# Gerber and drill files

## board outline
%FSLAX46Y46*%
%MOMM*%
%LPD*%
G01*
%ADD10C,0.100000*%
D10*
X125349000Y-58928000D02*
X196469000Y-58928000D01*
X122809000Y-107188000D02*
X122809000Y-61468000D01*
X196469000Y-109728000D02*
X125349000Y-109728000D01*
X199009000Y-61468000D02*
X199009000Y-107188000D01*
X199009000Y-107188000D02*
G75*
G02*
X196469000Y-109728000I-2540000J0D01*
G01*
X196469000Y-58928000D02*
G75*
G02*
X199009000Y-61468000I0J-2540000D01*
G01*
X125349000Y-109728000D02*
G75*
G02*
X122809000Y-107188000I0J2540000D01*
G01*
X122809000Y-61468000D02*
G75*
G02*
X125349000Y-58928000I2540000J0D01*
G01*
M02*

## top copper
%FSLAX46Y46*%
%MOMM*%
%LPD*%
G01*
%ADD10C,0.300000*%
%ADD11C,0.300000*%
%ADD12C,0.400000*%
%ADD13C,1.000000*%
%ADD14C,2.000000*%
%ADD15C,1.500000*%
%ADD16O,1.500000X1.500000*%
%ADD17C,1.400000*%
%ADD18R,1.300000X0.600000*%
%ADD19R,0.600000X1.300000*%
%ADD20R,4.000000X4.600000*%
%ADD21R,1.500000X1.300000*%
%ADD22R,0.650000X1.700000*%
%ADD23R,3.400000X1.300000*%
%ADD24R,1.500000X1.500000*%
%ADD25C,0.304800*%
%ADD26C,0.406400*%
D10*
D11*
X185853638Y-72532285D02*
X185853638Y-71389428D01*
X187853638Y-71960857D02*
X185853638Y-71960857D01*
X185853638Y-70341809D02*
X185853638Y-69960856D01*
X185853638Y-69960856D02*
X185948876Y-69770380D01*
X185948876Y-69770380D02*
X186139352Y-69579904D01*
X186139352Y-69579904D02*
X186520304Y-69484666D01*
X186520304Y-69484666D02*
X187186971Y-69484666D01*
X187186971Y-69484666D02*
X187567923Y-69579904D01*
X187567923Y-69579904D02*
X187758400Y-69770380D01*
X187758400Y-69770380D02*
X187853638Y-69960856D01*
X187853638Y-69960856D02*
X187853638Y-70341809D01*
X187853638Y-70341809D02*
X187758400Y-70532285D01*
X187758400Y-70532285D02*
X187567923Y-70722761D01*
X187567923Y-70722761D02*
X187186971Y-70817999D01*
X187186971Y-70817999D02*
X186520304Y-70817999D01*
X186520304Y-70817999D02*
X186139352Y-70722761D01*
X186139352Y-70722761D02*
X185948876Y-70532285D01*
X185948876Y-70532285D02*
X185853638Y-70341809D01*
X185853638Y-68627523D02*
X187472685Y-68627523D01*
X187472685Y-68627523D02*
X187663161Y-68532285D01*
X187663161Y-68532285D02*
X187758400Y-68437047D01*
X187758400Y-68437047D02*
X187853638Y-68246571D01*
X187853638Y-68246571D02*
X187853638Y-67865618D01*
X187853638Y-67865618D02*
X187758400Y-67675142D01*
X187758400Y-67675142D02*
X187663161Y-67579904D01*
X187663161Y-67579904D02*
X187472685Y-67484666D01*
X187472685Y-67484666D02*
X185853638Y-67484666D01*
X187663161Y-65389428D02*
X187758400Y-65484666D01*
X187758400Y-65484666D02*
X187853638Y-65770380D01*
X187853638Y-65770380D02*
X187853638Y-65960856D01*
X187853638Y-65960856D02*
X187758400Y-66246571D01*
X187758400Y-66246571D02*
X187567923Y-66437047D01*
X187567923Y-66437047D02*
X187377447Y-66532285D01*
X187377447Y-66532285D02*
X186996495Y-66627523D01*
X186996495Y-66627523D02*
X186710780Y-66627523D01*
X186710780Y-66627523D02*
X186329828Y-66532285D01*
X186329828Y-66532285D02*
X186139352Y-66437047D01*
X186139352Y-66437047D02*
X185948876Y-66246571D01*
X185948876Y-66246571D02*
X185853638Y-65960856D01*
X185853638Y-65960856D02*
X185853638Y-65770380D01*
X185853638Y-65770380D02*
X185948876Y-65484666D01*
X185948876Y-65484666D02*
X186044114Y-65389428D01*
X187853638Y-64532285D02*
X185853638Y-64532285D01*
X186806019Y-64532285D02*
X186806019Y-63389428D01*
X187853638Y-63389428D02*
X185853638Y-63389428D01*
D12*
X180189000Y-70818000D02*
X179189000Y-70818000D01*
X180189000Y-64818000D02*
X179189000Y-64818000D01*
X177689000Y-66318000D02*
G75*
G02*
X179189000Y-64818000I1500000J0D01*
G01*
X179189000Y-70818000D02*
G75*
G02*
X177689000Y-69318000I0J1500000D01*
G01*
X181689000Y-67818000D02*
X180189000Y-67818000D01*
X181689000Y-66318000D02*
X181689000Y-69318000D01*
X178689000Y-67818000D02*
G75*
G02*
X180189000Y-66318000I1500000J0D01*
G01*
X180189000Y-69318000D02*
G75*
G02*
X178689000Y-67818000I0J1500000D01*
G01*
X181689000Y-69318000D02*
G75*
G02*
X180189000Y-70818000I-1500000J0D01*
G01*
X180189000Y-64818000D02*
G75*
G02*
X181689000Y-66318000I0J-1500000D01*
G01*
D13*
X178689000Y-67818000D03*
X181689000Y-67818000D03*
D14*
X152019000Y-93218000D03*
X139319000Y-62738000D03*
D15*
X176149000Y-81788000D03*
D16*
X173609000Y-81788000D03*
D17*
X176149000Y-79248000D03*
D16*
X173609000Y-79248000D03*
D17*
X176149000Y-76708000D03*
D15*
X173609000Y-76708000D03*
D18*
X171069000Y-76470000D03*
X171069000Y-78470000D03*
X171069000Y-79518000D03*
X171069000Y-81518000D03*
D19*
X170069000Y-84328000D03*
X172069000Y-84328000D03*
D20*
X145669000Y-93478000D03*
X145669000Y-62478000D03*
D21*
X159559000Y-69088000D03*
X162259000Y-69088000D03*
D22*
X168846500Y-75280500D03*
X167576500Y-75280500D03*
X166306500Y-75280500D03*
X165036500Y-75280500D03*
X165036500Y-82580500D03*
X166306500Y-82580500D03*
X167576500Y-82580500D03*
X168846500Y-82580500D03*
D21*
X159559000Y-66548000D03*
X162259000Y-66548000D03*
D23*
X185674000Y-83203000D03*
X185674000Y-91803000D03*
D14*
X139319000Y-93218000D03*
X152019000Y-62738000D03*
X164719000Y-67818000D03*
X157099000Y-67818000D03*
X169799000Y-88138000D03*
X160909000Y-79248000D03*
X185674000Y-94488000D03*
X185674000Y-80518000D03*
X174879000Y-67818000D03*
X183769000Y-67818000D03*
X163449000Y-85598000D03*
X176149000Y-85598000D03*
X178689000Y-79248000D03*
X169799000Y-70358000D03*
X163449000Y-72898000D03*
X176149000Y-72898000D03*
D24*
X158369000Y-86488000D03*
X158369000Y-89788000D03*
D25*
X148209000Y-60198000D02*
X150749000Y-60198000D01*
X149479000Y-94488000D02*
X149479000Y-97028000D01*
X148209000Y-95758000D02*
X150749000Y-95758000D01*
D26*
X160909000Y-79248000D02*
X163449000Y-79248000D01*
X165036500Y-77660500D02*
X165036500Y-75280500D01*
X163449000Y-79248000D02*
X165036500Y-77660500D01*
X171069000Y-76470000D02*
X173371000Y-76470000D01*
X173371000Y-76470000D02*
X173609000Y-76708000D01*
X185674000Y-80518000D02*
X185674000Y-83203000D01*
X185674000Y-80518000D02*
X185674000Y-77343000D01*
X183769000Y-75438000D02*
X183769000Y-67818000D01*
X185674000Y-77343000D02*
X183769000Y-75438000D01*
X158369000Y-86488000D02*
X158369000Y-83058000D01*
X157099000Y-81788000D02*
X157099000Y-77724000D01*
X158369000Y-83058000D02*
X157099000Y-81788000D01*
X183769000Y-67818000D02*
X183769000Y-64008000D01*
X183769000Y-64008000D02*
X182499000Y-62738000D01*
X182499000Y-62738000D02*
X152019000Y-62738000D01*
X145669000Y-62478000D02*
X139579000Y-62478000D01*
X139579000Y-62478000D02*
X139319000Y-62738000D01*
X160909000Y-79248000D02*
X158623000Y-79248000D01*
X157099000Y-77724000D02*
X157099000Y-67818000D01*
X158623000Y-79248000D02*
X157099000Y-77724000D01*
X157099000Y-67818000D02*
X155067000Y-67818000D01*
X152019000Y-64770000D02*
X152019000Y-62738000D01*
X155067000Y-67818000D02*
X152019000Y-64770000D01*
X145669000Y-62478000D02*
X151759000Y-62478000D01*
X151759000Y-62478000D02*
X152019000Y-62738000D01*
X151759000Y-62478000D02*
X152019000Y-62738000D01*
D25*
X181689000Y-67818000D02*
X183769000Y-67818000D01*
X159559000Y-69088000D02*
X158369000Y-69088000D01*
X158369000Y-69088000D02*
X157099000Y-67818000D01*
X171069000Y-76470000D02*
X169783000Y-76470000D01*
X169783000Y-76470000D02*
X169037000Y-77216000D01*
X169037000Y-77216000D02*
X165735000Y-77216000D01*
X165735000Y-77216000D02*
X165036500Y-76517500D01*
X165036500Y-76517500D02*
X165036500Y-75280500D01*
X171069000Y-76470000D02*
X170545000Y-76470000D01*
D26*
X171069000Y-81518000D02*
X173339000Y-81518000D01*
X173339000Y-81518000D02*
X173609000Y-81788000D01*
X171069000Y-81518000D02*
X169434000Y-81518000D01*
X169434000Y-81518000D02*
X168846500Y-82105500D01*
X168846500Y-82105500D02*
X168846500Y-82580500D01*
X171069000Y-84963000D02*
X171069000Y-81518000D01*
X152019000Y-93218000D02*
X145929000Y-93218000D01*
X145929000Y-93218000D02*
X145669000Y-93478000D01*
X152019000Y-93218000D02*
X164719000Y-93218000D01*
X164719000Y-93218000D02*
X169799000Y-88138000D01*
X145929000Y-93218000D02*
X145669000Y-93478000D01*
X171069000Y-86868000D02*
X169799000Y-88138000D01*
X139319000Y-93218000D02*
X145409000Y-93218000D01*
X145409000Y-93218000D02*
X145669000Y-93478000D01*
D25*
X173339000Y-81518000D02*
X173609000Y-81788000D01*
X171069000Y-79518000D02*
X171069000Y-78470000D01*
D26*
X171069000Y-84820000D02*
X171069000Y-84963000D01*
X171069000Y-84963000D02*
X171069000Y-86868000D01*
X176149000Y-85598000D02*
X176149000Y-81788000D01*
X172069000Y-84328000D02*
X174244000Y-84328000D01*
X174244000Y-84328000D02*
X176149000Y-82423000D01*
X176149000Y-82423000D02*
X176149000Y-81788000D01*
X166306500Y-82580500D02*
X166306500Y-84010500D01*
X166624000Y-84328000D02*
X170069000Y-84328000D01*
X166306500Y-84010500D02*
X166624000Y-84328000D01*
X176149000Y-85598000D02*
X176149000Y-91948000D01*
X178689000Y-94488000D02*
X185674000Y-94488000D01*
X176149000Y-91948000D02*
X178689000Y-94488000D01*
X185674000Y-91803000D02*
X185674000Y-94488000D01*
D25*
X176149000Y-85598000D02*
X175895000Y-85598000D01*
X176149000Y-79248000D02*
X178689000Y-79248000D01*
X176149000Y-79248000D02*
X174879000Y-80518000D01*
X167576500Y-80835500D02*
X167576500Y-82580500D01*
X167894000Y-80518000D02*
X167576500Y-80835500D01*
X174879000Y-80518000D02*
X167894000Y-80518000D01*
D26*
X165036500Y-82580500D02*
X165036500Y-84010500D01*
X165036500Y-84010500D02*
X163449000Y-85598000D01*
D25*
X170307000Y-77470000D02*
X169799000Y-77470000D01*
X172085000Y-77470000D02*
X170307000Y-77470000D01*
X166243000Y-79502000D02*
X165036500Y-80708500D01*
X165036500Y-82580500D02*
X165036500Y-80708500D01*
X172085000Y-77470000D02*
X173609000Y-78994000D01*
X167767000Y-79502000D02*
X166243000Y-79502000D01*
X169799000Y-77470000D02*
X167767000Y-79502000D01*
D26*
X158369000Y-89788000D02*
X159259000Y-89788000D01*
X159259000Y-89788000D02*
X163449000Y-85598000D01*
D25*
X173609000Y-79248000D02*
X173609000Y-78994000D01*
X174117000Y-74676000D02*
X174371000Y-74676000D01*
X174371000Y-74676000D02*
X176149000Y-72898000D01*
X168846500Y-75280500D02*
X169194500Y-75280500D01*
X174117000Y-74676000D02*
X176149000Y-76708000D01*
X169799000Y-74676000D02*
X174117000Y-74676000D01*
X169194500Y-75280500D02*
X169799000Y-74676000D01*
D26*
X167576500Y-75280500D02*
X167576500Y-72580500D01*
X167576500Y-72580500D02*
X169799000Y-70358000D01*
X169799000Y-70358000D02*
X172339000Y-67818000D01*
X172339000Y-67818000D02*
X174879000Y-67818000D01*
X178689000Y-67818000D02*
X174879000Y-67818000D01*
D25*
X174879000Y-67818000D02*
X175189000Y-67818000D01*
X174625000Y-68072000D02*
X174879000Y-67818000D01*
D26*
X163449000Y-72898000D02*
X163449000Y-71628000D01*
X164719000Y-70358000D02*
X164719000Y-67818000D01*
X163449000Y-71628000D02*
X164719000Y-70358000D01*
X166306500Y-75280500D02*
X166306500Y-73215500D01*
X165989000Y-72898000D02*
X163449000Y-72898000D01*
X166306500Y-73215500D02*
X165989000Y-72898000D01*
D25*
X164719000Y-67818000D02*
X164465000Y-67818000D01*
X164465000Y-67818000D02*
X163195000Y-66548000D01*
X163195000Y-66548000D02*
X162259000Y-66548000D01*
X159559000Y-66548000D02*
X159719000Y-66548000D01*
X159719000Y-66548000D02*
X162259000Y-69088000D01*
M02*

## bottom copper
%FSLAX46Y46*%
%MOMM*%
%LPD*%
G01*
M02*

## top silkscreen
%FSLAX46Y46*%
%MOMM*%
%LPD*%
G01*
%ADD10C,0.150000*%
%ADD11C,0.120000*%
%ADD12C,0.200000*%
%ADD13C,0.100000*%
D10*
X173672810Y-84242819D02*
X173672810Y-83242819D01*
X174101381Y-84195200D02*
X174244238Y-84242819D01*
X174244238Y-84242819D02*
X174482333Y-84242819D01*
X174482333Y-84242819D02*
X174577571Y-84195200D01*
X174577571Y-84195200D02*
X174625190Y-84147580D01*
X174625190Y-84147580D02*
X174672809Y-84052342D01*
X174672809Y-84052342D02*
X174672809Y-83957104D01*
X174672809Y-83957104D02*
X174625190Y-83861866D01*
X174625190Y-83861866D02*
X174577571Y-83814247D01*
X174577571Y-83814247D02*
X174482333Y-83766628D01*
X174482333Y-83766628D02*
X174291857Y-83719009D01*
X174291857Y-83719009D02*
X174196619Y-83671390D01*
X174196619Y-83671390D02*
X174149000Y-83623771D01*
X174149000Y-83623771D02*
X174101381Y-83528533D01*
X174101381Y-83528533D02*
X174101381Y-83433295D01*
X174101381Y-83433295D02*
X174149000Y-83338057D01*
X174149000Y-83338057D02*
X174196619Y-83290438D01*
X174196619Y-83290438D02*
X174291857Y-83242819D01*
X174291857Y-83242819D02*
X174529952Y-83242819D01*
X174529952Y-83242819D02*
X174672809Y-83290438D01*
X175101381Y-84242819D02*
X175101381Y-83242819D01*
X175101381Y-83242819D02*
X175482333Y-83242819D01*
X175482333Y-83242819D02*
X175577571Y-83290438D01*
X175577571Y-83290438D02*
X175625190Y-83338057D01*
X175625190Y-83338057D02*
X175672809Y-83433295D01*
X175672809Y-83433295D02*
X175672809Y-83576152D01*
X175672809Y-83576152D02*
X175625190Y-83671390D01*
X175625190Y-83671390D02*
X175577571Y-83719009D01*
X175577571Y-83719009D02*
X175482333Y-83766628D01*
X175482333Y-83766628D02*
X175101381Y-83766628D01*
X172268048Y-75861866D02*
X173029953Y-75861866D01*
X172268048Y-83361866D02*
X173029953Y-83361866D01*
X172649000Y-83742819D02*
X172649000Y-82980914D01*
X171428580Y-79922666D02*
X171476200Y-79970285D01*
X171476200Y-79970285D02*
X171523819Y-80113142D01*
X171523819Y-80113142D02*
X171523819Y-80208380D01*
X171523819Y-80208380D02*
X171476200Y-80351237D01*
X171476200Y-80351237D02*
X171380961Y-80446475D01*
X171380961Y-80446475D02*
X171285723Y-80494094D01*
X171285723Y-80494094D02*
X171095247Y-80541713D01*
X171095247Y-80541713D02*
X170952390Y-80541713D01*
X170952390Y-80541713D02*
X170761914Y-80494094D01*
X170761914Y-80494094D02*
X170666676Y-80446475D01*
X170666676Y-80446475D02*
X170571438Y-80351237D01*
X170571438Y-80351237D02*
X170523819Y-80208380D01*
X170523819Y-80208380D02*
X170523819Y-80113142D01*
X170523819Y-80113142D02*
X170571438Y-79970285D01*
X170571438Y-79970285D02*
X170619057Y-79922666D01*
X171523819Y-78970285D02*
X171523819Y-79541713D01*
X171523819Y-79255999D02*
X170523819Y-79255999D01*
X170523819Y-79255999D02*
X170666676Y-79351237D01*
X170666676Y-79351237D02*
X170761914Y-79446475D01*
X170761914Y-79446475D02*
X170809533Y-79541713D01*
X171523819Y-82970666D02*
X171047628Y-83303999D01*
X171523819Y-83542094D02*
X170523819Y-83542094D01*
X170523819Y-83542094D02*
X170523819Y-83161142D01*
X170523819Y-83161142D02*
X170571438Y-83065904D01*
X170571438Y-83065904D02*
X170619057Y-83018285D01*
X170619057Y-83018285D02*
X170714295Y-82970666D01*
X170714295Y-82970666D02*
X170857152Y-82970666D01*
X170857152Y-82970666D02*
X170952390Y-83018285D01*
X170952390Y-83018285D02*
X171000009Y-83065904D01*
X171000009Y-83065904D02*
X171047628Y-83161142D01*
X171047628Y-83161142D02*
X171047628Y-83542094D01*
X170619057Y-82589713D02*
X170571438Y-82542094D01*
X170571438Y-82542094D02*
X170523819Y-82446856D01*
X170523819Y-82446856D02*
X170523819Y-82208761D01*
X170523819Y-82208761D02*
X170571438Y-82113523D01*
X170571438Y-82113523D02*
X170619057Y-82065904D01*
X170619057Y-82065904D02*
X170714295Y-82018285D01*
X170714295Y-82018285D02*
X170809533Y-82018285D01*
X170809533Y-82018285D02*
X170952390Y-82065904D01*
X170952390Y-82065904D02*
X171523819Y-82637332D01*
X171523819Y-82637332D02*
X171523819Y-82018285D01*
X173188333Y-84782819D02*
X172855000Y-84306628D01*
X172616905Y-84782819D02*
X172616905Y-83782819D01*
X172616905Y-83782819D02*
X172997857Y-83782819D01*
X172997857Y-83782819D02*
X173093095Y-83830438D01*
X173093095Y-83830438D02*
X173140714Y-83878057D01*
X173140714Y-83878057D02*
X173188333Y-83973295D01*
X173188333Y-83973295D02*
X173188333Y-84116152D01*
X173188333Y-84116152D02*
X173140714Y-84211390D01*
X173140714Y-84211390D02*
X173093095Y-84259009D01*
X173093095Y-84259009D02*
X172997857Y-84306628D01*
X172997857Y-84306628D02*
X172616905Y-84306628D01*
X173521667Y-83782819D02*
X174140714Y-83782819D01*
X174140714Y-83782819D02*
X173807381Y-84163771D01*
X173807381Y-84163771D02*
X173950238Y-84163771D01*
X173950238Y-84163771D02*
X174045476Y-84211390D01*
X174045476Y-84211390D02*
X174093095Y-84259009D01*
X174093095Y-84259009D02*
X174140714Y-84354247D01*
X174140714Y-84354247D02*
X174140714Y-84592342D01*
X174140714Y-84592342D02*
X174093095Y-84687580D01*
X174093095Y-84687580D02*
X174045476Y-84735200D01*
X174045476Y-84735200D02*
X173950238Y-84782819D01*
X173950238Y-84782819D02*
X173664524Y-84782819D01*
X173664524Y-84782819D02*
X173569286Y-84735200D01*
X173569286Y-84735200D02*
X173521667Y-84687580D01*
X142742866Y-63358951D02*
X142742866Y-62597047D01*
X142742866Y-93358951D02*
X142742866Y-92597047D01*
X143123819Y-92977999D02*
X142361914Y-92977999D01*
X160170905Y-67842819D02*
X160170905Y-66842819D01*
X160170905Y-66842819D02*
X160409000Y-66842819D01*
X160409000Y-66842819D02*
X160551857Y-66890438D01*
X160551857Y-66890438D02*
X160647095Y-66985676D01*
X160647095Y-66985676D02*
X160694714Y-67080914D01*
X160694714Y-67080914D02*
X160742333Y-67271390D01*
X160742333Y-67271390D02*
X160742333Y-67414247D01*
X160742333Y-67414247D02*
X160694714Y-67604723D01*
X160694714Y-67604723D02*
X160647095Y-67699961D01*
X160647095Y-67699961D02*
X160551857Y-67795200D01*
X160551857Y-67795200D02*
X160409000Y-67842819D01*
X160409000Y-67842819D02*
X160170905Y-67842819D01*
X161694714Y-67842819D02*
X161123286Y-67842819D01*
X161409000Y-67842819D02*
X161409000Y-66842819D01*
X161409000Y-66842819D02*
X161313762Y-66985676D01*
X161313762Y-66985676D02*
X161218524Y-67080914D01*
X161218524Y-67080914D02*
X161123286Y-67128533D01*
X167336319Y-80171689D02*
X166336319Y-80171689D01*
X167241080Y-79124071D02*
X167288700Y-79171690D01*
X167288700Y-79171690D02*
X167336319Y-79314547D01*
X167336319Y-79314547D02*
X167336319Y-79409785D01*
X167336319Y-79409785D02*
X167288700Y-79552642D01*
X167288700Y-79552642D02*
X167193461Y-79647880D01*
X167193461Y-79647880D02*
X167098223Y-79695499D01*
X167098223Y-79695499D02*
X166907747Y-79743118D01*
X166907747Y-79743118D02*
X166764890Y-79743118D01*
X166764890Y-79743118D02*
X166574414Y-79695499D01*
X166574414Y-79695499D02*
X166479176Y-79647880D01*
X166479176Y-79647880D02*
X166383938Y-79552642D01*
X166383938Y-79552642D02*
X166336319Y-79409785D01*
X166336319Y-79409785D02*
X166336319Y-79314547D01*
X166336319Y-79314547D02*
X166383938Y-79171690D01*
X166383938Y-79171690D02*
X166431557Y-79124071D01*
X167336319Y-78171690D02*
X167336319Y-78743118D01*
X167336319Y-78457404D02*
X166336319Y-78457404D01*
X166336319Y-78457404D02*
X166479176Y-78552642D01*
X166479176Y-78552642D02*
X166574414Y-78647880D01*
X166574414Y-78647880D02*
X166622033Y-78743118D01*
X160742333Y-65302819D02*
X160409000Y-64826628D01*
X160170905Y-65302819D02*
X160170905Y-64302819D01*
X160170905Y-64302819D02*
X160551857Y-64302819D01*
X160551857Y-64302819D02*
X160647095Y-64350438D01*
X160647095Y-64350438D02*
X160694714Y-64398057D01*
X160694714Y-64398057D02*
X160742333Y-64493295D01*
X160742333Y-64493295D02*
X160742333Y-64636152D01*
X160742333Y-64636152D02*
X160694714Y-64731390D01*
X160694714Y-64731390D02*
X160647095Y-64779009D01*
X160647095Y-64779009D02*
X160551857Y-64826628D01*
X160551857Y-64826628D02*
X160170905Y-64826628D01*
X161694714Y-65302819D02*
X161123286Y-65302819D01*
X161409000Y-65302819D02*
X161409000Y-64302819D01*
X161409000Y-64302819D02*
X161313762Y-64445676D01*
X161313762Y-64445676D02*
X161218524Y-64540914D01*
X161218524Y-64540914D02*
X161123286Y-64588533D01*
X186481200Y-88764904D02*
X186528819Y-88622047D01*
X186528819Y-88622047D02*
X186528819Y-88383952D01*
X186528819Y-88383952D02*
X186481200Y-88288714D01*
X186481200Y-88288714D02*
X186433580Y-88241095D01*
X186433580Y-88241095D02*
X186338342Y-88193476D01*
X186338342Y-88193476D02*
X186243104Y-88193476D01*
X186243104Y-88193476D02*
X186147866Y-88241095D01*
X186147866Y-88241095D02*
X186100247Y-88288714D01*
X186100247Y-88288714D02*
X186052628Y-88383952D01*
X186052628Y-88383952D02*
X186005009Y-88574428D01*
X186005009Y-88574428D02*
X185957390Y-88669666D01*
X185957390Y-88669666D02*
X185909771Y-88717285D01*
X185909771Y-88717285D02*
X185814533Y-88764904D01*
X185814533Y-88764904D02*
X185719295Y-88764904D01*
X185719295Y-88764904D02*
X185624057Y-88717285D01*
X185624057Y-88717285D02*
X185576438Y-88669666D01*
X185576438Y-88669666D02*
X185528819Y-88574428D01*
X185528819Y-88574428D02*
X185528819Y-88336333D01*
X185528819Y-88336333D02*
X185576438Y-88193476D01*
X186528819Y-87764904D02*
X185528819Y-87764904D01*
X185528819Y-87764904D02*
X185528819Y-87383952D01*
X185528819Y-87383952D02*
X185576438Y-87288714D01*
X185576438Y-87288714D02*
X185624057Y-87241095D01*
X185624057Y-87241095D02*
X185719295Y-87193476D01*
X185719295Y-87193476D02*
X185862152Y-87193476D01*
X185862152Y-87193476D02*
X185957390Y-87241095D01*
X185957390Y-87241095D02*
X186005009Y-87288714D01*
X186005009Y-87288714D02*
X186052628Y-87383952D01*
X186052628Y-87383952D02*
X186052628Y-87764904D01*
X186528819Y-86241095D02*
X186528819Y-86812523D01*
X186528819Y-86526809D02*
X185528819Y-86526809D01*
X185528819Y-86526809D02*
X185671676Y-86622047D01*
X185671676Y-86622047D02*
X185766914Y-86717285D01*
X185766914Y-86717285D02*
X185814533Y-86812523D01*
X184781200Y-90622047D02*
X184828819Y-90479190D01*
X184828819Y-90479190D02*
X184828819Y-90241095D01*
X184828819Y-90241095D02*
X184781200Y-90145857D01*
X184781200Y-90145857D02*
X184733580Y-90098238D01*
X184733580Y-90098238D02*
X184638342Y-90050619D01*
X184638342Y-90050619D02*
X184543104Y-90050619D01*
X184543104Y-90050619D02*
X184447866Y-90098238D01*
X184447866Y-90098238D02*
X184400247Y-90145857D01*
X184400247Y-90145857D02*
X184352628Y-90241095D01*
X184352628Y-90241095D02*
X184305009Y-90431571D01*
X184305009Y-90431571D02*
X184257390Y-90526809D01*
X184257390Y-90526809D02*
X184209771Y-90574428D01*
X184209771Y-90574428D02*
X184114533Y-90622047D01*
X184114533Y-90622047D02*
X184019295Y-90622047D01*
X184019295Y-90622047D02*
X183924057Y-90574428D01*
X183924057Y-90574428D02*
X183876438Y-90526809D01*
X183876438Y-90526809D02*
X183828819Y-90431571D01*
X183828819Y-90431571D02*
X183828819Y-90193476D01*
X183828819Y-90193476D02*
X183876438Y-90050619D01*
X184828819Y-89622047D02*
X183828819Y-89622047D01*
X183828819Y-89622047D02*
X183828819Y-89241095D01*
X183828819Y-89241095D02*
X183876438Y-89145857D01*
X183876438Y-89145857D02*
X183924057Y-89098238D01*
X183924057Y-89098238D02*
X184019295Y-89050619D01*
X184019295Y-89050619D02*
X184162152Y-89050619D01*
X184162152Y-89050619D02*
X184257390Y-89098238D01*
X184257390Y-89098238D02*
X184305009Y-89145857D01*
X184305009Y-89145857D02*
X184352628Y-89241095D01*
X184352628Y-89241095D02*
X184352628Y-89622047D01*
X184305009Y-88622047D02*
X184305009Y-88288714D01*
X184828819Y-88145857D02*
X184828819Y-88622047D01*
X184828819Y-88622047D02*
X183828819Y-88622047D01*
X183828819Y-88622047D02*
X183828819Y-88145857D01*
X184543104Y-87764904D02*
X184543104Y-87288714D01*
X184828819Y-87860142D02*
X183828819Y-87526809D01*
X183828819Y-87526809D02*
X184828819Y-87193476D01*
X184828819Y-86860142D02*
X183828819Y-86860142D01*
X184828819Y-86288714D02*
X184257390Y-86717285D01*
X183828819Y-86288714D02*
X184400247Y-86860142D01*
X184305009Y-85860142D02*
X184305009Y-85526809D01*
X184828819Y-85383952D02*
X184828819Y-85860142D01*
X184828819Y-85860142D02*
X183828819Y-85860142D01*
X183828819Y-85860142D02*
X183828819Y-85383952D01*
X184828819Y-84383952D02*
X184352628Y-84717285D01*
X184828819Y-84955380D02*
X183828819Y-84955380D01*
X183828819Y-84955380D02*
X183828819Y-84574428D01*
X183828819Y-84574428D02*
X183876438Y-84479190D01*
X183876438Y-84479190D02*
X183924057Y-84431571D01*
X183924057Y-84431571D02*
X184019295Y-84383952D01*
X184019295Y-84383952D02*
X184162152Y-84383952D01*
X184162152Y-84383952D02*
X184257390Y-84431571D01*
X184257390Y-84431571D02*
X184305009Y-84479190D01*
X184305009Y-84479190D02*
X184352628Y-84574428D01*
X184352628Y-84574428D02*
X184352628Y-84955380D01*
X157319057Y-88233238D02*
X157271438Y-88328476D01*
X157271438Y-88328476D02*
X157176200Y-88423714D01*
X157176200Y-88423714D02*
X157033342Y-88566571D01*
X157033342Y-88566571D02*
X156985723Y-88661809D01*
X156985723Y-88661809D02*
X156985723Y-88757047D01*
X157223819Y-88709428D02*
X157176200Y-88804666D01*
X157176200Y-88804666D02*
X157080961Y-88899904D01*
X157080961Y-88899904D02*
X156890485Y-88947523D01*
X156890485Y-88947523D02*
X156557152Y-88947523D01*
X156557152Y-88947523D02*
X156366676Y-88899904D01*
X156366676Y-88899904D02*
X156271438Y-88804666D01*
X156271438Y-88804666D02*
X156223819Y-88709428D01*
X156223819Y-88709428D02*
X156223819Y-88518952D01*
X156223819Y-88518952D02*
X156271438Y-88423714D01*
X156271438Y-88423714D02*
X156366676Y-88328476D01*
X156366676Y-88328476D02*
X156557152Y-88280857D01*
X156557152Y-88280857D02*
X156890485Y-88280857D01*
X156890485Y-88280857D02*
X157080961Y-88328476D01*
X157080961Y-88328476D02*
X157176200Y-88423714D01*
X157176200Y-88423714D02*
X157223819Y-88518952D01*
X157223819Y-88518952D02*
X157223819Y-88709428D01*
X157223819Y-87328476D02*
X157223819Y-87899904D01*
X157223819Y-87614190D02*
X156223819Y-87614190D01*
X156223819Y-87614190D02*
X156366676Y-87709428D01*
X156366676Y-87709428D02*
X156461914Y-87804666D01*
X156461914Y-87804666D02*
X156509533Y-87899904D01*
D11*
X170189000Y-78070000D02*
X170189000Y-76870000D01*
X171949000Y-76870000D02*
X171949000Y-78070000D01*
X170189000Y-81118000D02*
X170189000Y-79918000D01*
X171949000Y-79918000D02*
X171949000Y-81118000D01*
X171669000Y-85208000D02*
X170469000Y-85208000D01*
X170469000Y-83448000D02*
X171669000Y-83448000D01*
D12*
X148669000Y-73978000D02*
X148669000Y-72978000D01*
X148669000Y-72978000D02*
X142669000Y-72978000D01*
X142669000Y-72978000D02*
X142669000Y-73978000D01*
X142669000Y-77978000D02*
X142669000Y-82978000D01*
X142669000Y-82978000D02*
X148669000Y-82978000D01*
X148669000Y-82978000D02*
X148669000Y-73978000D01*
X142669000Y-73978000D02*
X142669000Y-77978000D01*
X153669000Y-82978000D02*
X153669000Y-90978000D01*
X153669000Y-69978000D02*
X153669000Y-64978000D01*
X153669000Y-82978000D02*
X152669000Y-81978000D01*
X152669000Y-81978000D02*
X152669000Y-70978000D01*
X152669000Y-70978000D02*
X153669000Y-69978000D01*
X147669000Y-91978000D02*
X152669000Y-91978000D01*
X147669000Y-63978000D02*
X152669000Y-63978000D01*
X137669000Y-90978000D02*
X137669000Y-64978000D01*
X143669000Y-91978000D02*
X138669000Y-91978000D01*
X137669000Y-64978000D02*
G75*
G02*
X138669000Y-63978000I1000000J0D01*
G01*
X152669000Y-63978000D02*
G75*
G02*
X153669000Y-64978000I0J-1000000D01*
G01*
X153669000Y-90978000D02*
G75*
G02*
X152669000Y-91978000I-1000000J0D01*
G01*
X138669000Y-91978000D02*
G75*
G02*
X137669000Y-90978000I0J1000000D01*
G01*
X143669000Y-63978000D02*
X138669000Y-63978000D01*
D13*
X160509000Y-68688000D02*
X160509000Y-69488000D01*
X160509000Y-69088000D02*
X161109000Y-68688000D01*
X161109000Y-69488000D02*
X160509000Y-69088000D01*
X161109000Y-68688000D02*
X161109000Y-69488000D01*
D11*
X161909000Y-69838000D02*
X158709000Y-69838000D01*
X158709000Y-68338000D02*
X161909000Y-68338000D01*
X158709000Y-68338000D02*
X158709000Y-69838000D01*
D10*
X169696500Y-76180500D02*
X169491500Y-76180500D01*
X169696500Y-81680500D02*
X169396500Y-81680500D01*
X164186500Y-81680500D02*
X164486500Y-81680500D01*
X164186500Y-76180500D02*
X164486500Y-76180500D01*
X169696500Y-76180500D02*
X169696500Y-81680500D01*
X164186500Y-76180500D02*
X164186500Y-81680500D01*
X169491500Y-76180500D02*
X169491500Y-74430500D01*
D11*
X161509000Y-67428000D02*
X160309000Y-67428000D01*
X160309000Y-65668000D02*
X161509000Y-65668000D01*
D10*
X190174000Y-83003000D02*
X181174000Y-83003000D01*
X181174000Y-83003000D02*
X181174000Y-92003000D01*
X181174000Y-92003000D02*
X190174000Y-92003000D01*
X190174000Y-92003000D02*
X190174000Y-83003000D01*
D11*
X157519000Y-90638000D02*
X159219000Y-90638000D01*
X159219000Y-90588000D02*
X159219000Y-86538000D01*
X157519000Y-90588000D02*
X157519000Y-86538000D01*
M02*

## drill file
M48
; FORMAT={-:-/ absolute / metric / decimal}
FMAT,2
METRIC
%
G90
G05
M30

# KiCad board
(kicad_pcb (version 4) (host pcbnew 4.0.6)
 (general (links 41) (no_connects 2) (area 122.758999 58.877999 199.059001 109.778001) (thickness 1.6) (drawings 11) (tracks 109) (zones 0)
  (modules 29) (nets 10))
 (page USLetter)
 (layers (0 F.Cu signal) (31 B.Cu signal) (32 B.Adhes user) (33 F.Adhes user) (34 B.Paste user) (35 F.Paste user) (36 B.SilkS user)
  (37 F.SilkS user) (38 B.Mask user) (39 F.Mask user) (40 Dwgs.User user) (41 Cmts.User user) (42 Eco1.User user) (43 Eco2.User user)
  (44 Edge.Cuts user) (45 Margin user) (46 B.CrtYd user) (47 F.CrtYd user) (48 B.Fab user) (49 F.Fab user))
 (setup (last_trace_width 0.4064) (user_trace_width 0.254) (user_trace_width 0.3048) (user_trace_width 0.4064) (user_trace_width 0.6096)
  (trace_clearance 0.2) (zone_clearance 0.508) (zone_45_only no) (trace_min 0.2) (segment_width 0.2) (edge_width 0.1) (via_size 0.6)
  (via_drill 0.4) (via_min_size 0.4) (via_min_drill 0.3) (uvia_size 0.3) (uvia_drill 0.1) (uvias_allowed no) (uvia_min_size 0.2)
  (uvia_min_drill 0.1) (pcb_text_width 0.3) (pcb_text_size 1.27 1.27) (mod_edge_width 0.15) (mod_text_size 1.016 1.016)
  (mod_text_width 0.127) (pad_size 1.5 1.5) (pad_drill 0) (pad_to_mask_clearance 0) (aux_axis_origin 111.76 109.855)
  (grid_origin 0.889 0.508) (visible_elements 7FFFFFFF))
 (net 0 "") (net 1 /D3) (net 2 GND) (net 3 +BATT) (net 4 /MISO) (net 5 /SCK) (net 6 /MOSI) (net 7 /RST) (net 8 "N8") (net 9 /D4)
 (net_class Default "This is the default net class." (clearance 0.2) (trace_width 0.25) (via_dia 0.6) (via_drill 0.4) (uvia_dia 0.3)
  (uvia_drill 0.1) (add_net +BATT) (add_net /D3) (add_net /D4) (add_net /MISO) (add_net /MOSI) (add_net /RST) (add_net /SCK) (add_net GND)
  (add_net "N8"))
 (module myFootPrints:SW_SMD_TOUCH (layer F.Cu) (at 178.689 67.818 270)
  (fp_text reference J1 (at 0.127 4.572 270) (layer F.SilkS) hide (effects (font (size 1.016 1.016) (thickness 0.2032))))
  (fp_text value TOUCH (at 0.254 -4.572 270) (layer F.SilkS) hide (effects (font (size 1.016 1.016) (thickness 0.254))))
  (fp_line (start 3 -1.5) (end 3 -0.5) (layer F.Cu) (width 0.4))
  (fp_line (start -3 -1.5) (end -3 -0.5) (layer F.Cu) (width 0.4))
  (fp_arc (start -1.5 -0.5) (end -1.5 1) (angle 90) (layer F.Cu) (width 0.4))
  (fp_arc (start 1.5 -0.5) (end 3 -0.5) (angle 90) (layer F.Cu) (width 0.4)) (fp_line (start 0 -3) (end 0 -1.5) (layer F.Cu) (width 0.4))
  (fp_line (start -1.5 -3) (end 1.5 -3) (layer F.Cu) (width 0.4))
  (fp_arc (start 0 -1.5) (end 0 0) (angle 90) (layer F.Cu) (width 0.4))
  (fp_arc (start 0 -1.5) (end 1.5 -1.5) (angle 90) (layer F.Cu) (width 0.4))
  (fp_arc (start 1.5 -1.5) (end 1.5 -3) (angle 90) (layer F.Cu) (width 0.4))
  (fp_arc (start -1.5 -1.5) (end -3 -1.5) (angle 90) (layer F.Cu) (width 0.4))
  (pad 2 smd circle (at 0 0 270) (size 1 1) (layers F.Cu) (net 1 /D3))
  (pad 1 smd circle (at 0 -3 270) (size 1 1) (layers F.Cu) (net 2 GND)))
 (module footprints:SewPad (layer F.Cu) (at 152.019 93.218)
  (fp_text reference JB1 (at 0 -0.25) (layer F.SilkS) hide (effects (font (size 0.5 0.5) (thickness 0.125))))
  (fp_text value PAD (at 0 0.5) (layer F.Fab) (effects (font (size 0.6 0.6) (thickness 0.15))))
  (pad 1 smd circle (at 0 0) (size 2 2) (layers F.Cu F.Mask) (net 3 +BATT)))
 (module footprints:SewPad (layer F.Cu) (at 139.319 62.738)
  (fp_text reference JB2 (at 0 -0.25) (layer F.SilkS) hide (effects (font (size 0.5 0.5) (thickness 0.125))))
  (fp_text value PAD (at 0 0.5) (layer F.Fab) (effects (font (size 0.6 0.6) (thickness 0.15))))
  (pad 1 smd circle (at 0 0) (size 2 2) (layers F.Cu F.Mask) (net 2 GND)))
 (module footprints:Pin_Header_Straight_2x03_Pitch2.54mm (layer F.Cu) (at 176.149 81.788 180)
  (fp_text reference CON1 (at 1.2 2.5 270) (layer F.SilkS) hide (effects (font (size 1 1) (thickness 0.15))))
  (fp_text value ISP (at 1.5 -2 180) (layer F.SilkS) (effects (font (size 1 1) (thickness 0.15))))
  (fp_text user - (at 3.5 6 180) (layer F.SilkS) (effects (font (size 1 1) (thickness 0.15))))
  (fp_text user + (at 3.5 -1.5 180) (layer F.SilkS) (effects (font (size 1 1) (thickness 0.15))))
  (pad 1 smd circle (at 0 0 180) (size 1.5 1.5) (layers F.Cu) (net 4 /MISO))
  (pad 2 smd oval (at 2.54 0 180) (size 1.5 1.5) (layers F.Cu) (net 3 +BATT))
  (pad 3 smd circle (at 0 2.54 180) (size 1.4 1.4) (layers F.Cu) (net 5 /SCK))
  (pad 4 smd oval (at 2.54 2.54 180) (size 1.5 1.5) (layers F.Cu) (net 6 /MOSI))
  (pad 5 smd circle (at 0 5.08 180) (size 1.4 1.4) (layers F.Cu) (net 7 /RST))
  (pad 6 smd circle (at 2.54 5.08 180) (size 1.5 1.5) (layers F.Cu) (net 2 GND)))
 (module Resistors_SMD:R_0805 (layer F.Cu) (at 171.069 77.47 270)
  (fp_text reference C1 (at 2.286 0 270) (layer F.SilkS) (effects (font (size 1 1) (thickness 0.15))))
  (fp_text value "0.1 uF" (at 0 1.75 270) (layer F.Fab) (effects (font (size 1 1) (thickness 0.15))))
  (fp_line (start 0.6 0.88) (end -0.6 0.88) (layer F.SilkS) (width 0.12))
  (fp_line (start -0.6 -0.88) (end 0.6 -0.88) (layer F.SilkS) (width 0.12))
  (pad 1 smd rect (at -1 0 270) (size 0.6 1.3) (layers F.Cu F.Paste F.Mask) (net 2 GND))
  (pad 2 smd rect (at 1 0 270) (size 0.6 1.3) (layers F.Cu F.Paste F.Mask) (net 3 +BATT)))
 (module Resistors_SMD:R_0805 (layer F.Cu) (at 171.069 80.518 270)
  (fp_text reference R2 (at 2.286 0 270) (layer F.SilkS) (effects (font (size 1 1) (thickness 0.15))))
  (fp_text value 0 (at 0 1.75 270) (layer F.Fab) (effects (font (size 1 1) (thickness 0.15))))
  (fp_line (start 0.6 0.88) (end -0.6 0.88) (layer F.SilkS) (width 0.12))
  (fp_line (start -0.6 -0.88) (end 0.6 -0.88) (layer F.SilkS) (width 0.12))
  (pad 1 smd rect (at -1 0 270) (size 0.6 1.3) (layers F.Cu F.Paste F.Mask) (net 3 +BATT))
  (pad 2 smd rect (at 1 0 270) (size 0.6 1.3) (layers F.Cu F.Paste F.Mask) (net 3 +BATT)))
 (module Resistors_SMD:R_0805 (layer F.Cu) (at 171.069 84.328)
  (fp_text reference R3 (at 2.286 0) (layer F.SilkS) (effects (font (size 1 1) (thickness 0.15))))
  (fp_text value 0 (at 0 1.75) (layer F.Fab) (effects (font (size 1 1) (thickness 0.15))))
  (fp_line (start 0.6 0.88) (end -0.6 0.88) (layer F.SilkS) (width 0.12))
  (fp_line (start -0.6 -0.88) (end 0.6 -0.88) (layer F.SilkS) (width 0.12))
  (pad 1 smd rect (at -1 0) (size 0.6 1.3) (layers F.Cu F.Paste F.Mask) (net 4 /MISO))
  (pad 2 smd rect (at 1 0) (size 0.6 1.3) (layers F.Cu F.Paste F.Mask) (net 4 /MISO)))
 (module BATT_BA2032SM (layer F.Cu) (at 145.669 77.978 90)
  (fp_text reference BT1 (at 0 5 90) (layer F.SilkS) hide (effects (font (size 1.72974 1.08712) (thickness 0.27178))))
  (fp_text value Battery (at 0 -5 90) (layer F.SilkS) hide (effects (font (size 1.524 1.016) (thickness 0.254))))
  (fp_line (start 4 3) (end 5 3) (layer F.SilkS) (width 0.2)) (fp_line (start 5 3) (end 5 -3) (layer F.SilkS) (width 0.2))
  (fp_line (start 5 -3) (end 4 -3) (layer F.SilkS) (width 0.2))
  (fp_line (start 0 -3) (end -5 -3) (layer F.SilkS) (width 0.2))
  (fp_line (start -5 -3) (end -5 3) (layer F.SilkS) (width 0.2)) (fp_line (start -5 3) (end 4 3) (layer F.SilkS) (width 0.2))
  (fp_line (start 4 -3) (end 0 -3) (layer F.SilkS) (width 0.2))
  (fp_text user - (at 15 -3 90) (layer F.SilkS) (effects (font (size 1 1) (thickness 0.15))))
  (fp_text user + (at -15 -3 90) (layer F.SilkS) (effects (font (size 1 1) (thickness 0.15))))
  (fp_line (start -5 8) (end -13 8) (layer F.SilkS) (width 0.2)) (fp_line (start 8 8) (end 13 8) (layer F.SilkS) (width 0.2))
  (fp_line (start -5 8) (end -4 7) (layer F.SilkS) (width 0.2)) (fp_line (start -4 7) (end 7 7) (layer F.SilkS) (width 0.2))
  (fp_line (start 7 7) (end 8 8) (layer F.SilkS) (width 0.2))
  (fp_line (start -14 2) (end -14 7) (layer F.SilkS) (width 0.2))
  (fp_line (start 14 2) (end 14 7) (layer F.SilkS) (width 0.2))
  (fp_line (start -13 -8) (end 13 -8) (layer F.SilkS) (width 0.2))
  (fp_line (start -14 -2) (end -14 -7) (layer F.SilkS) (width 0.2))
  (fp_arc (start 13 -7) (end 13 -8) (angle 90) (layer F.SilkS) (width 0.2))
  (fp_arc (start 13 7) (end 14 7) (angle 90) (layer F.SilkS) (width 0.2))
  (fp_arc (start -13 7) (end -13 8) (angle 90) (layer F.SilkS) (width 0.2))
  (fp_arc (start -13 -7) (end -14 -7) (angle 90) (layer F.SilkS) (width 0.2))
  (fp_line (start 14 -2) (end 14 -7) (layer F.SilkS) (width 0.2))
  (pad 1 smd rect (at -15.5 0 90) (size 4.6 4) (layers F.Cu F.Paste F.Mask) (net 3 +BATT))
  (pad 2 smd rect (at 15.5 0 90) (size 4.6 4) (layers F.Cu F.Paste F.Mask) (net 2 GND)))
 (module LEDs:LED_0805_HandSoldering (layer F.Cu) (at 160.909 69.088)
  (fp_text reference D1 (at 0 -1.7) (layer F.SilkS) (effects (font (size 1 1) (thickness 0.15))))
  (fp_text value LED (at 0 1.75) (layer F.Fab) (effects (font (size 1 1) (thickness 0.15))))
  (fp_line (start -0.4 -0.4) (end -0.4 0.4) (layer F.SilkS) (width 0.1))
  (fp_line (start -0.4 0) (end 0.2 -0.4) (layer F.SilkS) (width 0.1))
  (fp_line (start 0.2 0.4) (end -0.4 0) (layer F.SilkS) (width 0.1))
  (fp_line (start 0.2 -0.4) (end 0.2 0.4) (layer F.SilkS) (width 0.1))
  (fp_line (start 1 0.75) (end -2.2 0.75) (layer F.SilkS) (width 0.12))
  (fp_line (start -2.2 -0.75) (end 1 -0.75) (layer F.SilkS) (width 0.12))
  (fp_line (start -2.2 -0.75) (end -2.2 0.75) (layer F.SilkS) (width 0.12))
  (pad 1 smd rect (at -1.35 0) (size 1.5 1.3) (layers F.Cu F.Paste F.Mask) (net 2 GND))
  (pad 2 smd rect (at 1.35 0) (size 1.5 1.3) (layers F.Cu F.Paste F.Mask) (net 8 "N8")))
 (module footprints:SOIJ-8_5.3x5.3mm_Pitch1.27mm (layer F.Cu) (at 166.9415 78.9305 270)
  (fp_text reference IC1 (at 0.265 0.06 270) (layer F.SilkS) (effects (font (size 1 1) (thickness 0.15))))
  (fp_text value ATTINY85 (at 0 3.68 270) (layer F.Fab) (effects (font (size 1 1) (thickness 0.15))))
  (fp_line (start -2.75 -2.755) (end -2.75 -2.55) (layer F.SilkS) (width 0.15))
  (fp_line (start 2.75 -2.755) (end 2.75 -2.455) (layer F.SilkS) (width 0.15))
  (fp_line (start 2.75 2.755) (end 2.75 2.455) (layer F.SilkS) (width 0.15))
  (fp_line (start -2.75 2.755) (end -2.75 2.455) (layer F.SilkS) (width 0.15))
  (fp_line (start -2.75 -2.755) (end 2.75 -2.755) (layer F.SilkS) (width 0.15))
  (fp_line (start -2.75 2.755) (end 2.75 2.755) (layer F.SilkS) (width 0.15))
  (fp_line (start -2.75 -2.55) (end -4.5 -2.55) (layer F.SilkS) (width 0.15))
  (pad 1 smd rect (at -3.65 -1.905 270) (size 1.7 0.65) (layers F.Cu F.Paste F.Mask) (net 7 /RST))
  (pad 2 smd rect (at -3.65 -0.635 270) (size 1.7 0.65) (layers F.Cu F.Paste F.Mask) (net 1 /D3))
  (pad 3 smd rect (at -3.65 0.635 270) (size 1.7 0.65) (layers F.Cu F.Paste F.Mask) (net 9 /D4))
  (pad 4 smd rect (at -3.65 1.905 270) (size 1.7 0.65) (layers F.Cu F.Paste F.Mask) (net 2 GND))
  (pad 5 smd rect (at 3.65 1.905 270) (size 1.7 0.65) (layers F.Cu F.Paste F.Mask) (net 6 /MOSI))
  (pad 6 smd rect (at 3.65 0.635 270) (size 1.7 0.65) (layers F.Cu F.Paste F.Mask) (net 4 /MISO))
  (pad 7 smd rect (at 3.65 -0.635 270) (size 1.7 0.65) (layers F.Cu F.Paste F.Mask) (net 5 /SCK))
  (pad 8 smd rect (at 3.65 -1.905 270) (size 1.7 0.65) (layers F.Cu F.Paste F.Mask) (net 3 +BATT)))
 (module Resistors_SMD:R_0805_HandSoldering (layer F.Cu) (at 160.909 66.548)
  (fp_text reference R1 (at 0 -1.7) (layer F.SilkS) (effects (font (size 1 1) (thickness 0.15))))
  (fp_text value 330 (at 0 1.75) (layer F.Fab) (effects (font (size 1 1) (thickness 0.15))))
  (fp_line (start 0.6 0.88) (end -0.6 0.88) (layer F.SilkS) (width 0.12))
  (fp_line (start -0.6 -0.88) (end 0.6 -0.88) (layer F.SilkS) (width 0.12))
  (pad 1 smd rect (at -1.35 0) (size 1.5 1.3) (layers F.Cu F.Paste F.Mask) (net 8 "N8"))
  (pad 2 smd rect (at 1.35 0) (size 1.5 1.3) (layers F.Cu F.Paste F.Mask) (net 9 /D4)))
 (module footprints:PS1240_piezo (layer F.Cu) (at 185.674 87.503 270)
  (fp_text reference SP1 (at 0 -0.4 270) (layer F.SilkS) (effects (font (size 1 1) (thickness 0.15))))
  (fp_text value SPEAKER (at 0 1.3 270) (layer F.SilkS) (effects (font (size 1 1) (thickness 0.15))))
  (fp_line (start -4.5 -4.5) (end -4.5 4.5) (layer F.SilkS) (width 0.15))
  (fp_line (start -4.5 4.5) (end 4.5 4.5) (layer F.SilkS) (width 0.15))
  (fp_line (start 4.5 4.5) (end 4.5 -4.5) (layer F.SilkS) (width 0.15))
  (fp_line (start 4.5 -4.5) (end -4.5 -4.5) (layer F.SilkS) (width 0.15))
  (pad 1 smd rect (at -4.3 0 270) (size 1.3 3.4) (layers F.Cu F.Paste F.Mask) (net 2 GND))
  (pad 2 smd rect (at 4.3 0 270) (size 1.3 3.4) (layers F.Cu F.Paste F.Mask) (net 4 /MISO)))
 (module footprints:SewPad (layer F.Cu) (at 139.319 93.218)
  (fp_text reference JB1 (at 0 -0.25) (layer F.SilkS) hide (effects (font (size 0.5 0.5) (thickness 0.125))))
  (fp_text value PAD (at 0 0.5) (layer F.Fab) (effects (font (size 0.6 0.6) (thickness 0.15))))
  (pad 1 smd circle (at 0 0) (size 2 2) (layers F.Cu F.Mask) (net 3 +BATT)))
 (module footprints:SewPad (layer F.Cu) (at 152.019 62.738)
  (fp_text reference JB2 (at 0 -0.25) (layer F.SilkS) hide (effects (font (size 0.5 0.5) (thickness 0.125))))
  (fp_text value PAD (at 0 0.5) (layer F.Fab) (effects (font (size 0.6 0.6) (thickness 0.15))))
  (pad 1 smd circle (at 0 0) (size 2 2) (layers F.Cu F.Mask) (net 2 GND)))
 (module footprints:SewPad (layer F.Cu) (at 164.719 67.818)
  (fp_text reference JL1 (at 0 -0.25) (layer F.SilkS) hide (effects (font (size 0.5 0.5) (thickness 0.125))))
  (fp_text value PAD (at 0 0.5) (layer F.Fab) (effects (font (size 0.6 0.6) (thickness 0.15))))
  (pad 1 smd circle (at 0 0) (size 2 2) (layers F.Cu F.Mask) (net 9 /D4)))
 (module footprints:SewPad (layer F.Cu) (at 157.099 67.818)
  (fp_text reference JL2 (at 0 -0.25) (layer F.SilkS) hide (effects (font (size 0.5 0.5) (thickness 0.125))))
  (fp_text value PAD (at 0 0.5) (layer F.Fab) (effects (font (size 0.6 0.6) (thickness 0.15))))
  (pad 1 smd circle (at 0 0) (size 2 2) (layers F.Cu F.Mask) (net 2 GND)))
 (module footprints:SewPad (layer F.Cu) (at 169.799 88.138)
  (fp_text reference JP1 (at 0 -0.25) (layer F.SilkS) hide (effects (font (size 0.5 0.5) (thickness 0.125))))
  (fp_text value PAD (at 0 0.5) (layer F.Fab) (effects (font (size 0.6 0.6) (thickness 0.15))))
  (pad 1 smd circle (at 0 0) (size 2 2) (layers F.Cu F.Mask) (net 3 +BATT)))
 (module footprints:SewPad (layer F.Cu) (at 160.909 79.248)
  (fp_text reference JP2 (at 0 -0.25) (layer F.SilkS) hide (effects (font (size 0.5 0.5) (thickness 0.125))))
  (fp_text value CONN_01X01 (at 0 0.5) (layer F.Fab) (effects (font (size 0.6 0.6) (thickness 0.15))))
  (pad 1 smd circle (at 0 0) (size 2 2) (layers F.Cu F.Mask) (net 2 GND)))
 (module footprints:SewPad (layer F.Cu) (at 185.674 94.488)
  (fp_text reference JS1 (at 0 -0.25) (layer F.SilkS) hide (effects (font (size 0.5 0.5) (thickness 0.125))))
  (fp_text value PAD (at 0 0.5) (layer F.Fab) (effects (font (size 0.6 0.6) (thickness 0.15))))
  (pad 1 smd circle (at 0 0) (size 2 2) (layers F.Cu F.Mask) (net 4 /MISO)))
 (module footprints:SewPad (layer F.Cu) (at 185.674 80.518)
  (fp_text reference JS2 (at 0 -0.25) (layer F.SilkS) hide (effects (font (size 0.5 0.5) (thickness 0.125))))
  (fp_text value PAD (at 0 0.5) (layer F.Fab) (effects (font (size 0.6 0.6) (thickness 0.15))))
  (pad 1 smd circle (at 0 0) (size 2 2) (layers F.Cu F.Mask) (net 2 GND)))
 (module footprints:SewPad (layer F.Cu) (at 174.879 67.818)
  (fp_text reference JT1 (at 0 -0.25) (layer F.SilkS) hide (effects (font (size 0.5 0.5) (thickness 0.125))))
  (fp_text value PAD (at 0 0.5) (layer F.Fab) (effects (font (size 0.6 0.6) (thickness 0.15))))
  (pad 1 smd circle (at 0 0) (size 2 2) (layers F.Cu F.Mask) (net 1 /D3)))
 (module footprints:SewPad (layer F.Cu) (at 183.769 67.818)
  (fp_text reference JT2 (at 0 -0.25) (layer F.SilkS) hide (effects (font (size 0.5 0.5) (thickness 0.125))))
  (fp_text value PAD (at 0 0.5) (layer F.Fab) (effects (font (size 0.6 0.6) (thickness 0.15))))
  (pad 1 smd circle (at 0 0) (size 2 2) (layers F.Cu F.Mask) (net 2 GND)))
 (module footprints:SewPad (layer F.Cu) (at 163.449 85.598)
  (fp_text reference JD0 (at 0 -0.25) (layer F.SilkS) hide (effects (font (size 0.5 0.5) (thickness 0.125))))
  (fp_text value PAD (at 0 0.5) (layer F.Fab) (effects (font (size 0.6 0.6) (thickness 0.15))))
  (pad 1 smd circle (at 0 0) (size 2 2) (layers F.Cu F.Mask) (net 6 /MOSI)))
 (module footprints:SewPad (layer F.Cu) (at 176.149 85.598)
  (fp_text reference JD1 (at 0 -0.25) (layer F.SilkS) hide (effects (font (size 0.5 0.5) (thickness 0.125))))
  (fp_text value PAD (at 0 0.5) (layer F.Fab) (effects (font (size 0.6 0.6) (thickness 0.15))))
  (pad 1 smd circle (at 0 0) (size 2 2) (layers F.Cu F.Mask) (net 4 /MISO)))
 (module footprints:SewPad (layer F.Cu) (at 178.689 79.248)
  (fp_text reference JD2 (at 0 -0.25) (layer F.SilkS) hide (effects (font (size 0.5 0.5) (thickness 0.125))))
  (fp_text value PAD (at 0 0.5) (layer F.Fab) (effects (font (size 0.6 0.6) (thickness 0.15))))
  (pad 1 smd circle (at 0 0) (size 2 2) (layers F.Cu F.Mask) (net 5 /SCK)))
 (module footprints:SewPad (layer F.Cu) (at 169.799 70.358)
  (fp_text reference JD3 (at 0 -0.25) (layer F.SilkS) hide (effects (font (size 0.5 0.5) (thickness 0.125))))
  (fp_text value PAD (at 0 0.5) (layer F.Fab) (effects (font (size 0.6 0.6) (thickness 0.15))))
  (pad 1 smd circle (at 0 0) (size 2 2) (layers F.Cu F.Mask) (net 1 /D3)))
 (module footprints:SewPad (layer F.Cu) (at 163.449 72.898)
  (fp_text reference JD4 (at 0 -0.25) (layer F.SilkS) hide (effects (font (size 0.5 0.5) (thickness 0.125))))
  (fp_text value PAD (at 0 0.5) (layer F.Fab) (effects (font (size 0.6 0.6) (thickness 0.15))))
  (pad 1 smd circle (at 0 0) (size 2 2) (layers F.Cu F.Mask) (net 9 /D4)))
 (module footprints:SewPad (layer F.Cu) (at 176.149 72.898)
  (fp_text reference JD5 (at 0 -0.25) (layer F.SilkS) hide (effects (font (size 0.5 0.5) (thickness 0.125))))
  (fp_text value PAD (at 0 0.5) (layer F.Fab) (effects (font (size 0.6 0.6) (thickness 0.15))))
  (pad 1 smd circle (at 0 0) (size 2 2) (layers F.Cu F.Mask) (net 7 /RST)))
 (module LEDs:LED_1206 (layer F.Cu) (at 158.369 88.138 90)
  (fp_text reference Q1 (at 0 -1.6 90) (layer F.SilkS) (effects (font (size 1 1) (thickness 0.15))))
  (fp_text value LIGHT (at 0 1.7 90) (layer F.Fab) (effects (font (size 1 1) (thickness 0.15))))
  (fp_line (start -2.5 -0.85) (end -2.5 0.85) (layer F.SilkS) (width 0.12))
  (fp_line (start -2.45 0.85) (end 1.6 0.85) (layer F.SilkS) (width 0.12))
  (fp_line (start -2.45 -0.85) (end 1.6 -0.85) (layer F.SilkS) (width 0.12))
  (pad 2 smd rect (at 1.65 0 270) (size 1.5 1.5) (layers F.Cu F.Paste F.Mask) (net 2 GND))
  (pad 1 smd rect (at -1.65 0 270) (size 1.5 1.5) (layers F.Cu F.Paste F.Mask) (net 6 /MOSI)))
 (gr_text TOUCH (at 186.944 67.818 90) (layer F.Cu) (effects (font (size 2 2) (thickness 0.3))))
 (gr_line (start 125.349 58.928) (end 196.469 58.928) (angle 90) (layer Edge.Cuts) (width 0.1))
 (gr_line (start 122.809 107.188) (end 122.809 61.468) (angle 90) (layer Edge.Cuts) (width 0.1))
 (gr_line (start 196.469 109.728) (end 125.349 109.728) (angle 90) (layer Edge.Cuts) (width 0.1))
 (gr_line (start 199.009 61.468) (end 199.009 107.188) (angle 90) (layer Edge.Cuts) (width 0.1))
 (gr_arc (start 196.469 107.188) (end 199.009 107.188) (angle 90) (layer Edge.Cuts) (width 0.1))
 (gr_arc (start 196.469 61.468) (end 196.469 58.928) (angle 90) (layer Edge.Cuts) (width 0.1))
 (gr_arc (start 125.349 107.188) (end 125.349 109.728) (angle 90) (layer Edge.Cuts) (width 0.1))
 (gr_arc (start 125.349 61.468) (end 122.809 61.468) (angle 90) (layer Edge.Cuts) (width 0.1))
 (segment (start 148.209 60.198) (end 150.749 60.198) (width 0.3048) (layer F.Cu) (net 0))
 (segment (start 149.479 94.488) (end 149.479 97.028) (width 0.3048) (layer F.Cu) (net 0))
 (segment (start 148.209 95.758) (end 150.749 95.758) (width 0.3048) (layer F.Cu) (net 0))
 (segment (start 160.909 79.248) (end 163.449 79.248) (width 0.4064) (layer F.Cu) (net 2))
 (segment (start 165.0365 77.6605) (end 165.0365 75.2805) (width 0.4064) (layer F.Cu) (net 2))
 (segment (start 163.449 79.248) (end 165.0365 77.6605) (width 0.4064) (layer F.Cu) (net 2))
 (segment (start 171.069 76.47) (end 173.371 76.47) (width 0.4064) (layer F.Cu) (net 2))
 (segment (start 173.371 76.47) (end 173.609 76.708) (width 0.4064) (layer F.Cu) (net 2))
 (segment (start 185.674 80.518) (end 185.674 83.203) (width 0.4064) (layer F.Cu) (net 2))
 (segment (start 185.674 80.518) (end 185.674 77.343) (width 0.4064) (layer F.Cu) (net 2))
 (segment (start 183.769 75.438) (end 183.769 67.818) (width 0.4064) (layer F.Cu) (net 2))
 (segment (start 185.674 77.343) (end 183.769 75.438) (width 0.4064) (layer F.Cu) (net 2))
 (segment (start 158.369 86.488) (end 158.369 83.058) (width 0.4064) (layer F.Cu) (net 2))
 (segment (start 157.099 81.788) (end 157.099 77.724) (width 0.4064) (layer F.Cu) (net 2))
 (segment (start 158.369 83.058) (end 157.099 81.788) (width 0.4064) (layer F.Cu) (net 2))
 (segment (start 183.769 67.818) (end 183.769 64.008) (width 0.4064) (layer F.Cu) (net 2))
 (segment (start 183.769 64.008) (end 182.499 62.738) (width 0.4064) (layer F.Cu) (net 2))
 (segment (start 182.499 62.738) (end 152.019 62.738) (width 0.4064) (layer F.Cu) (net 2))
 (segment (start 145.669 62.478) (end 139.579 62.478) (width 0.4064) (layer F.Cu) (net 2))
 (segment (start 139.579 62.478) (end 139.319 62.738) (width 0.4064) (layer F.Cu) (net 2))
 (segment (start 160.909 79.248) (end 158.623 79.248) (width 0.4064) (layer F.Cu) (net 2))
 (segment (start 157.099 77.724) (end 157.099 67.818) (width 0.4064) (layer F.Cu) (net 2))
 (segment (start 158.623 79.248) (end 157.099 77.724) (width 0.4064) (layer F.Cu) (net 2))
 (segment (start 157.099 67.818) (end 155.067 67.818) (width 0.4064) (layer F.Cu) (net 2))
 (segment (start 152.019 64.77) (end 152.019 62.738) (width 0.4064) (layer F.Cu) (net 2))
 (segment (start 155.067 67.818) (end 152.019 64.77) (width 0.4064) (layer F.Cu) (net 2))
 (segment (start 145.669 62.478) (end 151.759 62.478) (width 0.4064) (layer F.Cu) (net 2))
 (segment (start 151.759 62.478) (end 152.019 62.738) (width 0.4064) (layer F.Cu) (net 2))
 (segment (start 151.759 62.478) (end 152.019 62.738) (width 0.4064) (layer F.Cu) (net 2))
 (segment (start 181.689 67.818) (end 183.769 67.818) (width 0.3048) (layer F.Cu) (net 2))
 (segment (start 159.559 69.088) (end 158.369 69.088) (width 0.3048) (layer F.Cu) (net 2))
 (segment (start 158.369 69.088) (end 157.099 67.818) (width 0.3048) (layer F.Cu) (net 2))
 (segment (start 171.069 76.47) (end 169.783 76.47) (width 0.3048) (layer F.Cu) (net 2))
 (segment (start 169.783 76.47) (end 169.037 77.216) (width 0.3048) (layer F.Cu) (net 2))
 (segment (start 169.037 77.216) (end 165.735 77.216) (width 0.3048) (layer F.Cu) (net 2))
 (segment (start 165.735 77.216) (end 165.0365 76.5175) (width 0.3048) (layer F.Cu) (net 2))
 (segment (start 165.0365 76.5175) (end 165.0365 75.2805) (width 0.3048) (layer F.Cu) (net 2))
 (segment (start 171.069 76.47) (end 170.545 76.47) (width 0.3048) (layer F.Cu) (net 2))
 (segment (start 171.069 81.518) (end 173.339 81.518) (width 0.4064) (layer F.Cu) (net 3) (status C00000))
 (segment (start 173.339 81.518) (end 173.609 81.788) (width 0.4064) (layer F.Cu) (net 3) (status C00000))
 (segment (start 171.069 81.518) (end 169.434 81.518) (width 0.4064) (layer F.Cu) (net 3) (status 400000))
 (segment (start 169.434 81.518) (end 168.8465 82.1055) (width 0.4064) (layer F.Cu) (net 3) (status 800000))
 (segment (start 168.8465 82.1055) (end 168.8465 82.5805) (width 0.4064) (layer F.Cu) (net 3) (status C00000))
 (segment (start 171.069 84.963) (end 171.069 81.518) (width 0.4064) (layer F.Cu) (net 3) (status 800000))
 (segment (start 152.019 93.218) (end 145.929 93.218) (width 0.4064) (layer F.Cu) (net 3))
 (segment (start 145.929 93.218) (end 145.669 93.478) (width 0.4064) (layer F.Cu) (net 3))
 (segment (start 152.019 93.218) (end 164.719 93.218) (width 0.4064) (layer F.Cu) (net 3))
 (segment (start 164.719 93.218) (end 169.799 88.138) (width 0.4064) (layer F.Cu) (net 3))
 (segment (start 145.929 93.218) (end 145.669 93.478) (width 0.4064) (layer F.Cu) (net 3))
 (segment (start 171.069 86.868) (end 169.799 88.138) (width 0.4064) (layer F.Cu) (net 3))
 (segment (start 139.319 93.218) (end 145.409 93.218) (width 0.4064) (layer F.Cu) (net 3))
 (segment (start 145.409 93.218) (end 145.669 93.478) (width 0.4064) (layer F.Cu) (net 3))
 (segment (start 173.339 81.518) (end 173.609 81.788) (width 0.3048) (layer F.Cu) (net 3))
 (segment (start 171.069 79.518) (end 171.069 78.47) (width 0.3048) (layer F.Cu) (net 3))
 (segment (start 171.069 84.82) (end 171.069 84.963) (width 0.4064) (layer F.Cu) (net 3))
 (segment (start 171.069 84.963) (end 171.069 86.868) (width 0.4064) (layer F.Cu) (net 3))
 (segment (start 176.149 85.598) (end 176.149 81.788) (width 0.4064) (layer F.Cu) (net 4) (status C00000))
 (segment (start 172.069 84.328) (end 174.244 84.328) (width 0.4064) (layer F.Cu) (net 4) (status 400000))
 (segment (start 174.244 84.328) (end 176.149 82.423) (width 0.4064) (layer F.Cu) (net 4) (status 800000))
 (segment (start 176.149 82.423) (end 176.149 81.788) (width 0.4064) (layer F.Cu) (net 4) (status C00000))
 (segment (start 166.3065 82.5805) (end 166.3065 84.0105) (width 0.4064) (layer F.Cu) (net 4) (status 400000))
 (segment (start 166.624 84.328) (end 170.069 84.328) (width 0.4064) (layer F.Cu) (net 4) (status 800000))
 (segment (start 166.3065 84.0105) (end 166.624 84.328) (width 0.4064) (layer F.Cu) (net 4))
 (segment (start 176.149 85.598) (end 176.149 91.948) (width 0.4064) (layer F.Cu) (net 4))
 (segment (start 178.689 94.488) (end 185.674 94.488) (width 0.4064) (layer F.Cu) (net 4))
 (segment (start 176.149 91.948) (end 178.689 94.488) (width 0.4064) (layer F.Cu) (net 4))
 (segment (start 185.674 91.803) (end 185.674 94.488) (width 0.4064) (layer F.Cu) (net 4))
 (segment (start 176.149 85.598) (end 175.895 85.598) (width 0.3048) (layer F.Cu) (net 4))
 (segment (start 176.149 79.248) (end 178.689 79.248) (width 0.3048) (layer F.Cu) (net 5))
 (segment (start 176.149 79.248) (end 174.879 80.518) (width 0.3048) (layer F.Cu) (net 5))
 (segment (start 167.5765 80.8355) (end 167.5765 82.5805) (width 0.3048) (layer F.Cu) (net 5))
 (segment (start 167.894 80.518) (end 167.5765 80.8355) (width 0.3048) (layer F.Cu) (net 5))
 (segment (start 174.879 80.518) (end 167.894 80.518) (width 0.3048) (layer F.Cu) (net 5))
 (segment (start 165.0365 82.5805) (end 165.0365 84.0105) (width 0.4064) (layer F.Cu) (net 6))
 (segment (start 165.0365 84.0105) (end 163.449 85.598) (width 0.4064) (layer F.Cu) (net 6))
 (segment (start 170.307 77.47) (end 169.799 77.47) (width 0.3048) (layer F.Cu) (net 6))
 (segment (start 172.085 77.47) (end 170.307 77.47) (width 0.3048) (layer F.Cu) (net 6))
 (segment (start 166.243 79.502) (end 165.0365 80.7085) (width 0.3048) (layer F.Cu) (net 6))
 (segment (start 165.0365 82.5805) (end 165.0365 80.7085) (width 0.3048) (layer F.Cu) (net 6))
 (segment (start 172.085 77.47) (end 173.609 78.994) (width 0.3048) (layer F.Cu) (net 6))
 (segment (start 167.767 79.502) (end 166.243 79.502) (width 0.3048) (layer F.Cu) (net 6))
 (segment (start 169.799 77.47) (end 167.767 79.502) (width 0.3048) (layer F.Cu) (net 6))
 (segment (start 158.369 89.788) (end 159.259 89.788) (width 0.4064) (layer F.Cu) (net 6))
 (segment (start 159.259 89.788) (end 163.449 85.598) (width 0.4064) (layer F.Cu) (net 6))
 (segment (start 173.609 79.248) (end 173.609 78.994) (width 0.3048) (layer F.Cu) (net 6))
 (segment (start 174.117 74.676) (end 174.371 74.676) (width 0.3048) (layer F.Cu) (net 7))
 (segment (start 174.371 74.676) (end 176.149 72.898) (width 0.3048) (layer F.Cu) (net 7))
 (segment (start 168.8465 75.2805) (end 169.1945 75.2805) (width 0.3048) (layer F.Cu) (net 7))
 (segment (start 174.117 74.676) (end 176.149 76.708) (width 0.3048) (layer F.Cu) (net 7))
 (segment (start 169.799 74.676) (end 174.117 74.676) (width 0.3048) (layer F.Cu) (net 7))
 (segment (start 169.1945 75.2805) (end 169.799 74.676) (width 0.3048) (layer F.Cu) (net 7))
 (segment (start 167.5765 75.2805) (end 167.5765 72.5805) (width 0.4064) (layer F.Cu) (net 1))
 (segment (start 167.5765 72.5805) (end 169.799 70.358) (width 0.4064) (layer F.Cu) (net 1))
 (segment (start 169.799 70.358) (end 172.339 67.818) (width 0.4064) (layer F.Cu) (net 1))
 (segment (start 172.339 67.818) (end 174.879 67.818) (width 0.4064) (layer F.Cu) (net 1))
 (segment (start 178.689 67.818) (end 174.879 67.818) (width 0.4064) (layer F.Cu) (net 1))
 (segment (start 174.879 67.818) (end 175.189 67.818) (width 0.3048) (layer F.Cu) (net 1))
 (segment (start 174.625 68.072) (end 174.879 67.818) (width 0.3048) (layer F.Cu) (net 1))
 (segment (start 163.449 72.898) (end 163.449 71.628) (width 0.4064) (layer F.Cu) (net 9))
 (segment (start 164.719 70.358) (end 164.719 67.818) (width 0.4064) (layer F.Cu) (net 9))
 (segment (start 163.449 71.628) (end 164.719 70.358) (width 0.4064) (layer F.Cu) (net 9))
 (segment (start 166.3065 75.2805) (end 166.3065 73.2155) (width 0.4064) (layer F.Cu) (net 9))
 (segment (start 165.989 72.898) (end 163.449 72.898) (width 0.4064) (layer F.Cu) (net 9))
 (segment (start 166.3065 73.2155) (end 165.989 72.898) (width 0.4064) (layer F.Cu) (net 9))
 (segment (start 164.719 67.818) (end 164.465 67.818) (width 0.3048) (layer F.Cu) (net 9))
 (segment (start 164.465 67.818) (end 163.195 66.548) (width 0.3048) (layer F.Cu) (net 9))
 (segment (start 163.195 66.548) (end 162.259 66.548) (width 0.3048) (layer F.Cu) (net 9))
 (segment (start 159.559 66.548) (end 159.719 66.548) (width 0.3048) (layer F.Cu) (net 8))
 (segment (start 159.719 66.548) (end 162.259 69.088) (width 0.3048) (layer F.Cu) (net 8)))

